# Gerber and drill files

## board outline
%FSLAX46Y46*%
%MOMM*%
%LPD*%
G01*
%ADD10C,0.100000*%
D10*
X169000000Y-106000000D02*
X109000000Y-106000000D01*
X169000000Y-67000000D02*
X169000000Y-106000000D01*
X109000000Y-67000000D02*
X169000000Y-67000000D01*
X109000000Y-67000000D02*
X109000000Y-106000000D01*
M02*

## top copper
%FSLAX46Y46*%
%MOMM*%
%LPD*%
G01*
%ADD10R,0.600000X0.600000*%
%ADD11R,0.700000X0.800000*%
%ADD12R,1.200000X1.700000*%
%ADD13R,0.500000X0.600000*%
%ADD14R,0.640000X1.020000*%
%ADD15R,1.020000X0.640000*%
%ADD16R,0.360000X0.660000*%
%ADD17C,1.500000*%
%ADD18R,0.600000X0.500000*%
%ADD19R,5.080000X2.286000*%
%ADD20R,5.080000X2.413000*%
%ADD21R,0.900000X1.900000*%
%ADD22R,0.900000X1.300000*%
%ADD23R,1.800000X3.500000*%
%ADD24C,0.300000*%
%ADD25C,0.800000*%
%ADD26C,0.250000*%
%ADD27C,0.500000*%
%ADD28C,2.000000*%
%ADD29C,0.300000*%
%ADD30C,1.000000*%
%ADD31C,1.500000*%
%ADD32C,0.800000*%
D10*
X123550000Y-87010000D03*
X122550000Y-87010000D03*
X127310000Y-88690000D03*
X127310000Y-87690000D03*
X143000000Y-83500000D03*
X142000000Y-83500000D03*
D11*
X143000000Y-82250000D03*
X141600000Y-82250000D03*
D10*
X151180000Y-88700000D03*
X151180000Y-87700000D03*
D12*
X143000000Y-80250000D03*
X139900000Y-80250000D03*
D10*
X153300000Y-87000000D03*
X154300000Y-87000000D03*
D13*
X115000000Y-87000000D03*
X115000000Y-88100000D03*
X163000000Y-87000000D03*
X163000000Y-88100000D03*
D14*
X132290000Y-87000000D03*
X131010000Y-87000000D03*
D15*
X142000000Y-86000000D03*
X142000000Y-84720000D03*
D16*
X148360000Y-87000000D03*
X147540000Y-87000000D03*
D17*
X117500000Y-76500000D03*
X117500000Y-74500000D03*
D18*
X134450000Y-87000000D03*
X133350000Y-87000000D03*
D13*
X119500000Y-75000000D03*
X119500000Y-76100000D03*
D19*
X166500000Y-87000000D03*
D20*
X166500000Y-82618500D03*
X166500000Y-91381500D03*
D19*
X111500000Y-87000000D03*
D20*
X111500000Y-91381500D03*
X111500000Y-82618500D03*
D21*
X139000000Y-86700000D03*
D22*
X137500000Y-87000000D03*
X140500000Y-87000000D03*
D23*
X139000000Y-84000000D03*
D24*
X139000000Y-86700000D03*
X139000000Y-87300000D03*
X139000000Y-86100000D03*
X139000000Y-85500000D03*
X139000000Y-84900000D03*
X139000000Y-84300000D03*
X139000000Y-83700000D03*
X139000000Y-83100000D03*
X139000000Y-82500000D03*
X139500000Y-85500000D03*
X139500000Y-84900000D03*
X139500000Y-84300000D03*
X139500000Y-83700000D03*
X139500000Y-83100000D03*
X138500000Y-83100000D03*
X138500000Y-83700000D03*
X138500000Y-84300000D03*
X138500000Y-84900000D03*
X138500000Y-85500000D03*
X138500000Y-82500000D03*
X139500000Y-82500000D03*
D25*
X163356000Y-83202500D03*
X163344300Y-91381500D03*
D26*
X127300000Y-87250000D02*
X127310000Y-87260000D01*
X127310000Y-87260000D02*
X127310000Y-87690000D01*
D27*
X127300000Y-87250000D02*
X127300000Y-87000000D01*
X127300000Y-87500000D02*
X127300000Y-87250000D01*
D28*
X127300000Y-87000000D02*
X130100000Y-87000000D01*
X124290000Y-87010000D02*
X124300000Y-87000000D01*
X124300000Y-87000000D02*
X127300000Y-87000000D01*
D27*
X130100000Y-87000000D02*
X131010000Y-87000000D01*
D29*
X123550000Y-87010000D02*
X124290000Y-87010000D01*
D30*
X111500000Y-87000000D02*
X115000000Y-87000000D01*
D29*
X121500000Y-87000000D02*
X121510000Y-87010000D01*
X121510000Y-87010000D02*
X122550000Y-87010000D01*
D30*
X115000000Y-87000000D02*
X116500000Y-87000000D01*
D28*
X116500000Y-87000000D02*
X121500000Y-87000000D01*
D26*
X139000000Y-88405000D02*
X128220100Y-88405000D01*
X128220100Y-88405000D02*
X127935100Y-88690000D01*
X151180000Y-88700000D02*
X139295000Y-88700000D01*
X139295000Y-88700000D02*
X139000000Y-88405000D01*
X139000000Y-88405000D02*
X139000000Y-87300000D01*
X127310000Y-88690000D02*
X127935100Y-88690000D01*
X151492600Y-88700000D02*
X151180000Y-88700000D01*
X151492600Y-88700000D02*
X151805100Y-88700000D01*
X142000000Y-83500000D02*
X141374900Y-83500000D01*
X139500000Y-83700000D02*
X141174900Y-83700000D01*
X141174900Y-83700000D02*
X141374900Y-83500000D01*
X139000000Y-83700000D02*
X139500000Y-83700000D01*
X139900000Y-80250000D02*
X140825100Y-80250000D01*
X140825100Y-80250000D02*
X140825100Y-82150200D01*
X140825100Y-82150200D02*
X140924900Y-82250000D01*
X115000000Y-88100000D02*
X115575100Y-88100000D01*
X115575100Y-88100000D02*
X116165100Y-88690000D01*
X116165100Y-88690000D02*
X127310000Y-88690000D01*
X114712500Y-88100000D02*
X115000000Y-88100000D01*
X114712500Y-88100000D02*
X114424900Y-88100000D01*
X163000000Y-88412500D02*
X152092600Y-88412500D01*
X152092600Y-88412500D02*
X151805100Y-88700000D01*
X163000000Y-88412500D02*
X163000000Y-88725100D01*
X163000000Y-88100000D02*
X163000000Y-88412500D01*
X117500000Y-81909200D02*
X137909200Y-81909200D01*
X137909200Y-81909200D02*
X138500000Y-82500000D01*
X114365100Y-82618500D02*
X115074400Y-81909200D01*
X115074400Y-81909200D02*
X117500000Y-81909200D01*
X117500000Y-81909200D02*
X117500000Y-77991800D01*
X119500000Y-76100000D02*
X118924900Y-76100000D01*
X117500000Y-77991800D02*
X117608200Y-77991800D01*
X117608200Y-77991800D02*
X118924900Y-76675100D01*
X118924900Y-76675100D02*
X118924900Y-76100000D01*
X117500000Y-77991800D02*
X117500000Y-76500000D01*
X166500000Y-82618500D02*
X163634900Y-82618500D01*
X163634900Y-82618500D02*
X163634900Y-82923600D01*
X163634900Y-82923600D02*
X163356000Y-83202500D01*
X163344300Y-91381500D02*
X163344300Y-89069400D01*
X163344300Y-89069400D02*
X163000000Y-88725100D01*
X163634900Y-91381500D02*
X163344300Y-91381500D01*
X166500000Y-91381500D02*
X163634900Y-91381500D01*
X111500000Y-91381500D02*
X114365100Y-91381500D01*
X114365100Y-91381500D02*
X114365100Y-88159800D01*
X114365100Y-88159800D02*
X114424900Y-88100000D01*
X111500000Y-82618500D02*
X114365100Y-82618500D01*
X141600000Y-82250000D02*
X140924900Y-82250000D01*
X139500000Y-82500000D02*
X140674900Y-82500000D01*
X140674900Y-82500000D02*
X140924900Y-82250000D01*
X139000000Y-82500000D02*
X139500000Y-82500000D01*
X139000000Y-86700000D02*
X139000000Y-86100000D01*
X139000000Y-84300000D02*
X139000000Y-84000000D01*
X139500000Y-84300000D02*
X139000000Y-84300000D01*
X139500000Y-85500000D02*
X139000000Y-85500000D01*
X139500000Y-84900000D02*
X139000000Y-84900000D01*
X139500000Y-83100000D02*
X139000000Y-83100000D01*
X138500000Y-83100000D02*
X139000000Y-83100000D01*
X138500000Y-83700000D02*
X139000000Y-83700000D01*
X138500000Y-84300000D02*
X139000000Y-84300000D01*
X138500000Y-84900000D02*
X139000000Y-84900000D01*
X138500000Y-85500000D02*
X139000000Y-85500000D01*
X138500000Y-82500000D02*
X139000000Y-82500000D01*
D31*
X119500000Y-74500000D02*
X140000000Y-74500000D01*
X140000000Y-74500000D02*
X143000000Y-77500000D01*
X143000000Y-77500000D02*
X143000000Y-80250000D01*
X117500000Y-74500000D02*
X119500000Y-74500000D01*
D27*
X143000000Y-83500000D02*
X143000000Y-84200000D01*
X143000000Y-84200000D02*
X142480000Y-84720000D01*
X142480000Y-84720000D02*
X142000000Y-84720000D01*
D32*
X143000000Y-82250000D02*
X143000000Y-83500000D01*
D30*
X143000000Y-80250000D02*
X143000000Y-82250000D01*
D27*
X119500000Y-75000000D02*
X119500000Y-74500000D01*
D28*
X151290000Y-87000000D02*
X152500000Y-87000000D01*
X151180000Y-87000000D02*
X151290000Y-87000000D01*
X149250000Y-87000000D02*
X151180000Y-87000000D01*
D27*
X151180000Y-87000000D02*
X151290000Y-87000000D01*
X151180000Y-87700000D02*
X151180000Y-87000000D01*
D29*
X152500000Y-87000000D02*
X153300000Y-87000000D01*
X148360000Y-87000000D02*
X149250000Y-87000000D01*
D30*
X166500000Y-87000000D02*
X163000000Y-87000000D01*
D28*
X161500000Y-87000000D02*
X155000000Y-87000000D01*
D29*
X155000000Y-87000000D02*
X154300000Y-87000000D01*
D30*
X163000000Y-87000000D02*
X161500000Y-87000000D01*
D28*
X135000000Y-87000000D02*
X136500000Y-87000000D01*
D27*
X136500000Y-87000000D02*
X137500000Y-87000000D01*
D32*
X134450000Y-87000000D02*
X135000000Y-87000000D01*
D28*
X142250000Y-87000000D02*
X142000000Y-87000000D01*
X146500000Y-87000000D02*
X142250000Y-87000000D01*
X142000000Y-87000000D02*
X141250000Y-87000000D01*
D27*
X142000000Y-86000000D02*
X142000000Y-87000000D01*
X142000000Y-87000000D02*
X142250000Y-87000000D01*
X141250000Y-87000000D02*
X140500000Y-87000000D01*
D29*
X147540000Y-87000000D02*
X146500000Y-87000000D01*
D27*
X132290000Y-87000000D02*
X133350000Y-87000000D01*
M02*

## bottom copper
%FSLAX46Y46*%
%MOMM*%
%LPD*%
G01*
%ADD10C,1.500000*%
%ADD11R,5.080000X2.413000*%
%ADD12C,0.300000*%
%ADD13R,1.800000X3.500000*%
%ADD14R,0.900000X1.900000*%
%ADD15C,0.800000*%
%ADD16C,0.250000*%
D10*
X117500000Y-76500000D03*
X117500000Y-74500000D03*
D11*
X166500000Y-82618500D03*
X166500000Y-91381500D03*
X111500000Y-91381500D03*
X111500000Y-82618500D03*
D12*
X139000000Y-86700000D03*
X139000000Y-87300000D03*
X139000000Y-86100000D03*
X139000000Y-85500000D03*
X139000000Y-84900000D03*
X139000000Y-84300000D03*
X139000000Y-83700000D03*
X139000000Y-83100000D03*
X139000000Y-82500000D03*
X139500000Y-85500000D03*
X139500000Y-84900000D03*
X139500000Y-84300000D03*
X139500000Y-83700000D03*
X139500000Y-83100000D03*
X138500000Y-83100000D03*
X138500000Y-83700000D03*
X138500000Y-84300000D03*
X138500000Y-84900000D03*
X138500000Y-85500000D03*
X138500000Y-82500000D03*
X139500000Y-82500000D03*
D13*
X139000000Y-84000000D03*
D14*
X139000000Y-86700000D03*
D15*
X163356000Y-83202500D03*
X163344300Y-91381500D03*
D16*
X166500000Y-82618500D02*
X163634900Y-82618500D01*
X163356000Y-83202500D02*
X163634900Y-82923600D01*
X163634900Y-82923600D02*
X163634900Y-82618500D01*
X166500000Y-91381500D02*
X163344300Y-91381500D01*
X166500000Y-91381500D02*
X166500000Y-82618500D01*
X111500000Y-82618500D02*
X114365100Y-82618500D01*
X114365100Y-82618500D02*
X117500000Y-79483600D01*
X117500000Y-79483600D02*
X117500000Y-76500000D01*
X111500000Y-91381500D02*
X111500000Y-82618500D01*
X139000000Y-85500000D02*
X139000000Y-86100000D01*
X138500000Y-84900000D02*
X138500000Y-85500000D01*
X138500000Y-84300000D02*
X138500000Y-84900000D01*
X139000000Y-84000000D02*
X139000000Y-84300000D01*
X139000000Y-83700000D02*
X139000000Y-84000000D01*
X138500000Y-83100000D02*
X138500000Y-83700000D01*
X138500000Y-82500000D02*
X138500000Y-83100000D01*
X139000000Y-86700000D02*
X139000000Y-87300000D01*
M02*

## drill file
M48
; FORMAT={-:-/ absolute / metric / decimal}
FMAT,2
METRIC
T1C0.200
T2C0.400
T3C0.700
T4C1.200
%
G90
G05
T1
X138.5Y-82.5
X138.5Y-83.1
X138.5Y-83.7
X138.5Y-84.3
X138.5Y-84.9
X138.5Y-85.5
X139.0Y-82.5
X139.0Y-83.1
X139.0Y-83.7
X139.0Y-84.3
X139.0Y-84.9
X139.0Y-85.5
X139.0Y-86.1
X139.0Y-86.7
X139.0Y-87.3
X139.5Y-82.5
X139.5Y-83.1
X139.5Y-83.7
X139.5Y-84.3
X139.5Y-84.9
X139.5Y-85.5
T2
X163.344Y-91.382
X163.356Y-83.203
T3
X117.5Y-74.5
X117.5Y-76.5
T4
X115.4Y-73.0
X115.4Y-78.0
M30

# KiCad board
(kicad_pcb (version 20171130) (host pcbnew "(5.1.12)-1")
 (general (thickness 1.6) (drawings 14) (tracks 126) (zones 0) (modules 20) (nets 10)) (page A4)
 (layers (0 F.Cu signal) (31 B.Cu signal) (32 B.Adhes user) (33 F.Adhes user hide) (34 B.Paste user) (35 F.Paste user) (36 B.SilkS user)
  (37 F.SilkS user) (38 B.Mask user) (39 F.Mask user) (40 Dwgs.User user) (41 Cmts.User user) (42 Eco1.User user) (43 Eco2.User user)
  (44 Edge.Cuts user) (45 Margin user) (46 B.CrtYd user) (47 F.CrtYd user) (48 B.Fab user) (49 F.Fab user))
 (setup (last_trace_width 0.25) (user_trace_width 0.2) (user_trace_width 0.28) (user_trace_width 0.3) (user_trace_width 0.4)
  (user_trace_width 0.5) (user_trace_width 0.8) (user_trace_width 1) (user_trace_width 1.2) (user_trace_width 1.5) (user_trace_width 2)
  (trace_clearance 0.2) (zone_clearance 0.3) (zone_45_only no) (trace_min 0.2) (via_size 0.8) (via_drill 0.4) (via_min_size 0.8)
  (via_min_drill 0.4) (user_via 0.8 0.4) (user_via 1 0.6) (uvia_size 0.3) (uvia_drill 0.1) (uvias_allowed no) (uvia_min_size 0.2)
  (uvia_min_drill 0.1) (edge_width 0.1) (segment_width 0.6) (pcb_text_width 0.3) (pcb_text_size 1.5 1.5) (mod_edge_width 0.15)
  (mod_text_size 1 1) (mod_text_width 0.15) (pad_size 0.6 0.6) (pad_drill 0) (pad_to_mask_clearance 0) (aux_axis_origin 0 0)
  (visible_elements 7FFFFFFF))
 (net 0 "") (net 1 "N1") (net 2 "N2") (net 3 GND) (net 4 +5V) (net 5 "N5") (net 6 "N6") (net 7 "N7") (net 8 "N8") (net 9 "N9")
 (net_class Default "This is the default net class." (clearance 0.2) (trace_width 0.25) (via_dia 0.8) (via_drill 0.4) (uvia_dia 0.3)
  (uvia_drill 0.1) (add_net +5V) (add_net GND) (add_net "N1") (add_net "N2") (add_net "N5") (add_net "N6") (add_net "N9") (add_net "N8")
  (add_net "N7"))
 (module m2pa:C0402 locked (layer F.Cu) (at 123.55 87.01 180)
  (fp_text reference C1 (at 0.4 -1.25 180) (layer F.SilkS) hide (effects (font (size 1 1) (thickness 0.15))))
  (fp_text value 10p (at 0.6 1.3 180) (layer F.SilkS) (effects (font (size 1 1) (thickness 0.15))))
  (pad 1 smd rect (at 0 0 180) (size 0.6 0.6) (layers F.Cu F.Paste F.Mask) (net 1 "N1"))
  (pad 2 smd rect (at 1 0 180) (size 0.6 0.6) (layers F.Cu F.Paste F.Mask) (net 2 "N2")))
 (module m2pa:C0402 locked (layer F.Cu) (at 127.31 88.69 90)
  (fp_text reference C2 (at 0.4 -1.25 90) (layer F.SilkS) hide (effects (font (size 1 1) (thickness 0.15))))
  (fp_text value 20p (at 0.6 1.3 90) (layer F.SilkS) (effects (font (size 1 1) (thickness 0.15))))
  (pad 1 smd rect (at 0 0 90) (size 0.6 0.6) (layers F.Cu F.Paste F.Mask) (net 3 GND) (zone_connect 2))
  (pad 2 smd rect (at 1 0 90) (size 0.6 0.6) (layers F.Cu F.Paste F.Mask) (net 1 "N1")))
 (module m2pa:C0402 (layer F.Cu) (at 143 83.5 180)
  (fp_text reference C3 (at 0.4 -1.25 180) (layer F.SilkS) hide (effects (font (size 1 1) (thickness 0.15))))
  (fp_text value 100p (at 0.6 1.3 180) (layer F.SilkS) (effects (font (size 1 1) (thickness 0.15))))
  (pad 1 smd rect (at 0 0 180) (size 0.6 0.6) (layers F.Cu F.Paste F.Mask) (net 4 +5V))
  (pad 2 smd rect (at 1 0 180) (size 0.6 0.6) (layers F.Cu F.Paste F.Mask) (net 3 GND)))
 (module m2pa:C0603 (layer F.Cu) (at 143 82.25 180)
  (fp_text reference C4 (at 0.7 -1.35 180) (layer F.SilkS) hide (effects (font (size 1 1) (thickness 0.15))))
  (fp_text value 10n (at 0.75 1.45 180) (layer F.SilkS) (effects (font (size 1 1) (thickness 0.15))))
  (pad 1 smd rect (at 0 0 180) (size 0.7 0.8) (layers F.Cu F.Paste F.Mask) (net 4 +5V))
  (pad 2 smd rect (at 1.4 0 180) (size 0.7 0.8) (layers F.Cu F.Paste F.Mask) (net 3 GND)))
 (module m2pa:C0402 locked (layer F.Cu) (at 151.18 88.7 90)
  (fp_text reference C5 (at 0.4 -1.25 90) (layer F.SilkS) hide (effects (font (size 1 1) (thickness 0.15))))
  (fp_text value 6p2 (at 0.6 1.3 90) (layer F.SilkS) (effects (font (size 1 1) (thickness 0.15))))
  (pad 1 smd rect (at 0 0 90) (size 0.6 0.6) (layers F.Cu F.Paste F.Mask) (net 3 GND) (zone_connect 2))
  (pad 2 smd rect (at 1 0 90) (size 0.6 0.6) (layers F.Cu F.Paste F.Mask) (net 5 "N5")))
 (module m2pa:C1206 (layer F.Cu) (at 143 80.25 180)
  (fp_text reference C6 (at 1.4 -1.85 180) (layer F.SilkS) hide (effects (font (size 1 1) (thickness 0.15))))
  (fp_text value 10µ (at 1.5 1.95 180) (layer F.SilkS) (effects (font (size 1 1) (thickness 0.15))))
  (pad 1 smd rect (at 0 0 180) (size 1.2 1.7) (layers F.Cu F.Paste F.Mask) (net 4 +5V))
  (pad 2 smd rect (at 3.1 0 180) (size 1.2 1.7) (layers F.Cu F.Paste F.Mask) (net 3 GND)))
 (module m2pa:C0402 (layer F.Cu) (at 153.3 87)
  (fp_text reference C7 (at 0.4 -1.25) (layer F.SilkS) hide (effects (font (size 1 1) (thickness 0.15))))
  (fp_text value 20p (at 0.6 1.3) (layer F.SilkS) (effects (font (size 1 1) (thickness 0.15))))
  (pad 1 smd rect (at 0 0) (size 0.6 0.6) (layers F.Cu F.Paste F.Mask) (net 5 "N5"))
  (pad 2 smd rect (at 1 0) (size 0.6 0.6) (layers F.Cu F.Paste F.Mask) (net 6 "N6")))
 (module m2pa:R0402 (layer F.Cu) (at 115 87 270)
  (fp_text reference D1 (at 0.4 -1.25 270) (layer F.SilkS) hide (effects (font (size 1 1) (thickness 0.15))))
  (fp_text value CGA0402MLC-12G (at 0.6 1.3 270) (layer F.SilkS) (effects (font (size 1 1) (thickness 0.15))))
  (pad 1 smd rect (at 0 0 270) (size 0.6 0.5) (layers F.Cu F.Paste F.Mask) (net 2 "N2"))
  (pad 2 smd rect (at 1.1 0 270) (size 0.6 0.5) (layers F.Cu F.Paste F.Mask) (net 3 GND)))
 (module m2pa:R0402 (layer F.Cu) (at 163 87 270)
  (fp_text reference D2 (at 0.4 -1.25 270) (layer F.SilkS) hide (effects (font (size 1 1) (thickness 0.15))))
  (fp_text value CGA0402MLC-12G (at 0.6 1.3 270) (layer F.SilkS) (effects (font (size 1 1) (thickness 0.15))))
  (pad 1 smd rect (at 0 0 270) (size 0.6 0.5) (layers F.Cu F.Paste F.Mask) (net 6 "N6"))
  (pad 2 smd rect (at 1.1 0 270) (size 0.6 0.5) (layers F.Cu F.Paste F.Mask) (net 3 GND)))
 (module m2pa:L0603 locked (layer F.Cu) (at 132.29 87 180)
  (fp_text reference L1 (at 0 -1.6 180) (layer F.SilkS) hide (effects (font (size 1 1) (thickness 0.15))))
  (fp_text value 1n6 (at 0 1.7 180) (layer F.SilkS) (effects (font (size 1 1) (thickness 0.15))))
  (pad 1 smd rect (at 0 0 180) (size 0.64 1.02) (layers F.Cu F.Paste F.Mask) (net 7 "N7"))
  (pad 2 smd rect (at 1.28 0 180) (size 0.64 1.02) (layers F.Cu F.Paste F.Mask) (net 1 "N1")))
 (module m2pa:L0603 (layer F.Cu) (at 142 86 90)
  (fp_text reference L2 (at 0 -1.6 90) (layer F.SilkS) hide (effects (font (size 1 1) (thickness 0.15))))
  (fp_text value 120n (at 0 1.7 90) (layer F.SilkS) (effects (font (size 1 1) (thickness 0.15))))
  (pad 1 smd rect (at 0 0 90) (size 0.64 1.02) (layers F.Cu F.Paste F.Mask) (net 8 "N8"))
  (pad 2 smd rect (at 1.28 0 90) (size 0.64 1.02) (layers F.Cu F.Paste F.Mask) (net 4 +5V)))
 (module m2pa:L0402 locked (layer F.Cu) (at 148.36 87 180)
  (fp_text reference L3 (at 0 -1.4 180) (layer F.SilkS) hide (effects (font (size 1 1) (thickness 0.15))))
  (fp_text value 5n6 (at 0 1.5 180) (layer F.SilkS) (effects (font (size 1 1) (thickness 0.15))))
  (pad 1 smd rect (at 0 0 180) (size 0.36 0.66) (layers F.Cu F.Paste F.Mask) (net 5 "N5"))
  (pad 2 smd rect (at 0.82 0 180) (size 0.36 0.66) (layers F.Cu F.Paste F.Mask) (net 8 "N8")))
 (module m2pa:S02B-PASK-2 (layer F.Cu) (at 117.5 76.5 90)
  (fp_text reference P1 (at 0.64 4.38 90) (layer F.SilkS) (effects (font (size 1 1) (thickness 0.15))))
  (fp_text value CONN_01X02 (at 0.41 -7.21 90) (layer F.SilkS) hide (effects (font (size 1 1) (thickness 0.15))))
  (pad 1 thru_hole circle (at 0 0 90) (size 1.5 1.5) (drill 0.7) (layers *.Cu *.Mask F.SilkS) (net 3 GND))
  (pad 2 thru_hole circle (at 2 0 90) (size 1.5 1.5) (drill 0.7) (layers *.Cu *.Mask F.SilkS) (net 4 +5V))
  (pad "" np_thru_hole circle (at -1.5 -2.1 90) (size 1.2 1.2) (drill 1.2) (layers *.Cu *.Mask F.SilkS))
  (pad "" np_thru_hole circle (at 3.5 -2.1 90) (size 1.2 1.2) (drill 1.2) (layers *.Cu *.Mask F.SilkS)))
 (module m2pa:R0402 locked (layer F.Cu) (at 134.45 87 180)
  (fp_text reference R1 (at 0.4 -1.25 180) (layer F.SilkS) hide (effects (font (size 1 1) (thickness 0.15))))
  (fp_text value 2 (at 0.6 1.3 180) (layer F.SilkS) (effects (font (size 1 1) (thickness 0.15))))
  (pad 1 smd rect (at 0 0 180) (size 0.6 0.5) (layers F.Cu F.Paste F.Mask) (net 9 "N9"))
  (pad 2 smd rect (at 1.1 0 180) (size 0.6 0.5) (layers F.Cu F.Paste F.Mask) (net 7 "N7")))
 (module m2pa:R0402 (layer F.Cu) (at 119.5 75 270)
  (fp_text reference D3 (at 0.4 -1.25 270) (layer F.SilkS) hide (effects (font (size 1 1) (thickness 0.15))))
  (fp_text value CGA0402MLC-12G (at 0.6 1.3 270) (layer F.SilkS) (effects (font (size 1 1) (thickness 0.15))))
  (pad 1 smd rect (at 0 0 270) (size 0.6 0.5) (layers F.Cu F.Paste F.Mask) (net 4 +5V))
  (pad 2 smd rect (at 1.1 0 270) (size 0.6 0.5) (layers F.Cu F.Paste F.Mask) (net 3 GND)))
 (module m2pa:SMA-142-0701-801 (layer F.Cu) (at 166.5 87 270)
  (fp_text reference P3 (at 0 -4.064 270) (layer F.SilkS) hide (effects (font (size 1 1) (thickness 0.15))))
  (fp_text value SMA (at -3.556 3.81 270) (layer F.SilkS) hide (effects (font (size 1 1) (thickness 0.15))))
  (pad 1 smd rect (at 0 0 270) (size 2.286 5.08) (layers F.Cu F.Mask) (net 6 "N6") (zone_connect 2))
  (pad 2 smd rect (at -4.3815 0 270) (size 2.413 5.08) (layers F.Cu F.Mask) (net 3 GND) (zone_connect 2))
  (pad 3 smd rect (at 4.3815 0 270) (size 2.413 5.08) (layers F.Cu F.Mask) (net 3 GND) (zone_connect 2))
  (pad 4 smd rect (at -4.3815 0 270) (size 2.413 5.08) (layers B.Cu B.Mask) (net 3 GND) (zone_connect 2))
  (pad 5 smd rect (at 4.3815 0 270) (size 2.413 5.08) (layers B.Cu B.Mask) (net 3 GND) (zone_connect 2)))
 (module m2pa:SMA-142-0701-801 (layer F.Cu) (at 111.5 87 90)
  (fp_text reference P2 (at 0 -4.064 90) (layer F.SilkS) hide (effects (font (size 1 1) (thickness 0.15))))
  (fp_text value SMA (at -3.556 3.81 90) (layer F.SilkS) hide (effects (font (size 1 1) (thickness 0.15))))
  (pad 1 smd rect (at 0 0 90) (size 2.286 5.08) (layers F.Cu F.Mask) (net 2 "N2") (zone_connect 2))
  (pad 2 smd rect (at -4.3815 0 90) (size 2.413 5.08) (layers F.Cu F.Mask) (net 3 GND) (zone_connect 2))
  (pad 3 smd rect (at 4.3815 0 90) (size 2.413 5.08) (layers F.Cu F.Mask) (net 3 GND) (zone_connect 2))
  (pad 4 smd rect (at -4.3815 0 90) (size 2.413 5.08) (layers B.Cu B.Mask) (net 3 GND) (zone_connect 2))
  (pad 5 smd rect (at 4.3815 0 90) (size 2.413 5.08) (layers B.Cu B.Mask) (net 3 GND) (zone_connect 2)))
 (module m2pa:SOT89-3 (layer F.Cu) (at 139 87)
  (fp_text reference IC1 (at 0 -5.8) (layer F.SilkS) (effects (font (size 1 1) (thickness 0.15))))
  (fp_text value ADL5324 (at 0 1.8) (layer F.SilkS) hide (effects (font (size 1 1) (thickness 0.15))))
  (pad 2 smd rect (at 0 -0.3 180) (size 0.9 1.9) (layers F.Cu F.Paste F.Mask) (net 3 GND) (zone_connect 2))
  (pad 1 smd rect (at -1.5 0 180) (size 0.9 1.3) (layers F.Cu F.Paste F.Mask) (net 9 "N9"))
  (pad 3 smd rect (at 1.5 0 180) (size 0.9 1.3) (layers F.Cu F.Paste F.Mask) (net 8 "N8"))
  (pad 2 smd rect (at 0 -3 180) (size 1.8 3.5) (layers F.Cu F.Paste F.Mask) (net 3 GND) (zone_connect 2))
  (pad 2 thru_hole circle (at 0 -0.3 180) (size 0.3 0.3) (drill 0.2) (layers *.Cu F.SilkS F.Mask) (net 3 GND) (zone_connect 2))
  (pad 2 thru_hole circle (at 0 0.3 180) (size 0.3 0.3) (drill 0.2) (layers *.Cu F.SilkS F.Mask) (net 3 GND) (zone_connect 2))
  (pad 2 thru_hole circle (at 0 -0.9 180) (size 0.3 0.3) (drill 0.2) (layers *.Cu F.SilkS F.Mask) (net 3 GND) (zone_connect 2))
  (pad 2 thru_hole circle (at 0 -1.5 180) (size 0.3 0.3) (drill 0.2) (layers *.Cu F.SilkS F.Mask) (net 3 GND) (zone_connect 2))
  (pad 2 thru_hole circle (at 0 -2.1 180) (size 0.3 0.3) (drill 0.2) (layers *.Cu F.SilkS F.Mask) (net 3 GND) (zone_connect 2))
  (pad 2 thru_hole circle (at 0 -2.7 180) (size 0.3 0.3) (drill 0.2) (layers *.Cu F.SilkS F.Mask) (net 3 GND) (zone_connect 2))
  (pad 2 thru_hole circle (at 0 -3.3 180) (size 0.3 0.3) (drill 0.2) (layers *.Cu F.SilkS F.Mask) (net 3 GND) (zone_connect 2))
  (pad 2 thru_hole circle (at 0 -3.9 180) (size 0.3 0.3) (drill 0.2) (layers *.Cu F.SilkS F.Mask) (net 3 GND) (zone_connect 2))
  (pad 2 thru_hole circle (at 0 -4.5 180) (size 0.3 0.3) (drill 0.2) (layers *.Cu F.SilkS F.Mask) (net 3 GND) (zone_connect 2))
  (pad 2 thru_hole circle (at 0.5 -1.5 180) (size 0.3 0.3) (drill 0.2) (layers *.Cu F.SilkS F.Mask) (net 3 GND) (zone_connect 2))
  (pad 2 thru_hole circle (at 0.5 -2.1 180) (size 0.3 0.3) (drill 0.2) (layers *.Cu F.SilkS F.Mask) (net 3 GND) (zone_connect 2))
  (pad 2 thru_hole circle (at 0.5 -2.7 180) (size 0.3 0.3) (drill 0.2) (layers *.Cu F.SilkS F.Mask) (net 3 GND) (zone_connect 2))
  (pad 2 thru_hole circle (at 0.5 -3.3 180) (size 0.3 0.3) (drill 0.2) (layers *.Cu F.SilkS F.Mask) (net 3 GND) (zone_connect 2))
  (pad 2 thru_hole circle (at 0.5 -3.9 180) (size 0.3 0.3) (drill 0.2) (layers *.Cu F.SilkS F.Mask) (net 3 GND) (zone_connect 2))
  (pad 2 thru_hole circle (at -0.5 -3.9 180) (size 0.3 0.3) (drill 0.2) (layers *.Cu F.SilkS F.Mask) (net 3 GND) (zone_connect 2))
  (pad 2 thru_hole circle (at -0.5 -3.3 180) (size 0.3 0.3) (drill 0.2) (layers *.Cu F.SilkS F.Mask) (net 3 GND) (zone_connect 2))
  (pad 2 thru_hole circle (at -0.5 -2.7 180) (size 0.3 0.3) (drill 0.2) (layers *.Cu F.SilkS F.Mask) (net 3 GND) (zone_connect 2))
  (pad 2 thru_hole circle (at -0.5 -2.1 180) (size 0.3 0.3) (drill 0.2) (layers *.Cu F.SilkS F.Mask) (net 3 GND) (zone_connect 2))
  (pad 2 thru_hole circle (at -0.5 -1.5 180) (size 0.3 0.3) (drill 0.2) (layers *.Cu F.SilkS F.Mask) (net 3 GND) (zone_connect 2))
  (pad 2 thru_hole circle (at -0.5 -4.5 180) (size 0.3 0.3) (drill 0.2) (layers *.Cu F.SilkS F.Mask) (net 3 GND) (zone_connect 2))
  (pad 2 thru_hole circle (at 0.5 -4.5 180) (size 0.3 0.3) (drill 0.2) (layers *.Cu F.SilkS F.Mask) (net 3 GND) (zone_connect 2))
  (pad 2 smd rect (at 0 -3 180) (size 1.8 3.5) (layers B.Cu) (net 3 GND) (zone_connect 2))
  (pad 2 smd rect (at 0 -0.3 180) (size 0.9 1.9) (layers B.Cu) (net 3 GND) (zone_connect 2)))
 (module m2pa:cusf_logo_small (layer F.Cu) (at 116 98)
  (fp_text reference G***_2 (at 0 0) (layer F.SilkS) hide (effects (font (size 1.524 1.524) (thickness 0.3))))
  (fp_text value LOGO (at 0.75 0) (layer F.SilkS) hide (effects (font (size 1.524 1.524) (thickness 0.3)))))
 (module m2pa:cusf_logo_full (layer F.Cu) (at 140.5 87.5)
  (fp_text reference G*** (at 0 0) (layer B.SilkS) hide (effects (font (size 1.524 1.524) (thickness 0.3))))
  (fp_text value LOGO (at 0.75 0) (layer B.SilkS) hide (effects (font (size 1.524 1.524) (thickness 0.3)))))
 (gr_line (start 169 106) (end 109 106) (angle 90) (layer Edge.Cuts) (width 0.1))
 (gr_line (start 169 67) (end 169 106) (angle 90) (layer Edge.Cuts) (width 0.1))
 (gr_line (start 109 67) (end 169 67) (angle 90) (layer Edge.Cuts) (width 0.1))
 (gr_line (start 109 67) (end 109 106) (angle 90) (layer Edge.Cuts) (width 0.1))
 (segment (start 127.3 87.25) (end 127.31 87.26) (width 0.25) (layer F.Cu) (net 1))
 (segment (start 127.31 87.26) (end 127.31 87.69) (width 0.25) (layer F.Cu) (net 1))
 (segment (start 127.3 87.25) (end 127.3 87) (width 0.5) (layer F.Cu) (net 1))
 (segment (start 127.3 87.5) (end 127.3 87.25) (width 0.5) (layer F.Cu) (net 1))
 (segment (start 127.3 87) (end 130.1 87) (width 2) (layer F.Cu) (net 1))
 (segment (start 124.29 87.01) (end 124.3 87) (width 2) (layer F.Cu) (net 1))
 (segment (start 124.3 87) (end 127.3 87) (width 2) (layer F.Cu) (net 1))
 (segment (start 130.1 87) (end 131.01 87) (width 0.5) (layer F.Cu) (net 1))
 (segment (start 123.55 87.01) (end 124.29 87.01) (width 0.3) (layer F.Cu) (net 1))
 (segment (start 111.5 87) (end 115 87) (width 1) (layer F.Cu) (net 2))
 (segment (start 121.5 87) (end 121.51 87.01) (width 0.3) (layer F.Cu) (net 2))
 (segment (start 121.51 87.01) (end 122.55 87.01) (width 0.3) (layer F.Cu) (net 2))
 (segment (start 115 87) (end 116.5 87) (width 1) (layer F.Cu) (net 2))
 (segment (start 116.5 87) (end 121.5 87) (width 2) (layer F.Cu) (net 2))
 (segment (start 139 88.405) (end 128.2201 88.405) (width 0.25) (layer F.Cu) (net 3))
 (segment (start 128.2201 88.405) (end 127.9351 88.69) (width 0.25) (layer F.Cu) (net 3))
 (segment (start 151.18 88.7) (end 139.295 88.7) (width 0.25) (layer F.Cu) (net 3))
 (segment (start 139.295 88.7) (end 139 88.405) (width 0.25) (layer F.Cu) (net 3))
 (segment (start 139 88.405) (end 139 87.3) (width 0.25) (layer F.Cu) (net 3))
 (segment (start 127.31 88.69) (end 127.9351 88.69) (width 0.25) (layer F.Cu) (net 3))
 (segment (start 151.4926 88.7) (end 151.18 88.7) (width 0.25) (layer F.Cu) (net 3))
 (segment (start 151.4926 88.7) (end 151.8051 88.7) (width 0.25) (layer F.Cu) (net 3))
 (segment (start 142 83.5) (end 141.3749 83.5) (width 0.25) (layer F.Cu) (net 3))
 (segment (start 139.5 83.7) (end 141.1749 83.7) (width 0.25) (layer F.Cu) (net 3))
 (segment (start 141.1749 83.7) (end 141.3749 83.5) (width 0.25) (layer F.Cu) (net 3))
 (segment (start 139 83.7) (end 139.5 83.7) (width 0.25) (layer F.Cu) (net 3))
 (segment (start 139.9 80.25) (end 140.8251 80.25) (width 0.25) (layer F.Cu) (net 3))
 (segment (start 140.8251 80.25) (end 140.8251 82.1502) (width 0.25) (layer F.Cu) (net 3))
 (segment (start 140.8251 82.1502) (end 140.9249 82.25) (width 0.25) (layer F.Cu) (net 3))
 (segment (start 115 88.1) (end 115.5751 88.1) (width 0.25) (layer F.Cu) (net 3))
 (segment (start 115.5751 88.1) (end 116.1651 88.69) (width 0.25) (layer F.Cu) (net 3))
 (segment (start 116.1651 88.69) (end 127.31 88.69) (width 0.25) (layer F.Cu) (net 3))
 (segment (start 114.7125 88.1) (end 115 88.1) (width 0.25) (layer F.Cu) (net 3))
 (segment (start 114.7125 88.1) (end 114.4249 88.1) (width 0.25) (layer F.Cu) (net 3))
 (segment (start 163 88.4125) (end 152.0926 88.4125) (width 0.25) (layer F.Cu) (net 3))
 (segment (start 152.0926 88.4125) (end 151.8051 88.7) (width 0.25) (layer F.Cu) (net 3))
 (segment (start 163 88.4125) (end 163 88.7251) (width 0.25) (layer F.Cu) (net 3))
 (segment (start 163 88.1) (end 163 88.4125) (width 0.25) (layer F.Cu) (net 3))
 (segment (start 117.5 81.9092) (end 137.9092 81.9092) (width 0.25) (layer F.Cu) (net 3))
 (segment (start 137.9092 81.9092) (end 138.5 82.5) (width 0.25) (layer F.Cu) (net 3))
 (segment (start 114.3651 82.6185) (end 115.0744 81.9092) (width 0.25) (layer F.Cu) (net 3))
 (segment (start 115.0744 81.9092) (end 117.5 81.9092) (width 0.25) (layer F.Cu) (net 3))
 (segment (start 117.5 81.9092) (end 117.5 77.9918) (width 0.25) (layer F.Cu) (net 3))
 (segment (start 119.5 76.1) (end 118.9249 76.1) (width 0.25) (layer F.Cu) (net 3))
 (segment (start 117.5 77.9918) (end 117.6082 77.9918) (width 0.25) (layer F.Cu) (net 3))
 (segment (start 117.6082 77.9918) (end 118.9249 76.6751) (width 0.25) (layer F.Cu) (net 3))
 (segment (start 118.9249 76.6751) (end 118.9249 76.1) (width 0.25) (layer F.Cu) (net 3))
 (segment (start 117.5 77.9918) (end 117.5 76.5) (width 0.25) (layer F.Cu) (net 3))
 (segment (start 166.5 82.6185) (end 163.6349 82.6185) (width 0.25) (layer F.Cu) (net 3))
 (segment (start 166.5 82.6185) (end 163.6349 82.6185) (width 0.25) (layer B.Cu) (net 3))
 (segment (start 163.6349 82.6185) (end 163.6349 82.9236) (width 0.25) (layer F.Cu) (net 3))
 (segment (start 163.6349 82.9236) (end 163.356 83.2025) (width 0.25) (layer F.Cu) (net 3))
 (segment (start 163.356 83.2025) (end 163.6349 82.9236) (width 0.25) (layer B.Cu) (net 3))
 (segment (start 163.6349 82.9236) (end 163.6349 82.6185) (width 0.25) (layer B.Cu) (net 3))
 (segment (start 163.3443 91.3815) (end 163.3443 89.0694) (width 0.25) (layer F.Cu) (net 3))
 (segment (start 163.3443 89.0694) (end 163 88.7251) (width 0.25) (layer F.Cu) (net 3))
 (segment (start 163.6349 91.3815) (end 163.3443 91.3815) (width 0.25) (layer F.Cu) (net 3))
 (segment (start 166.5 91.3815) (end 163.3443 91.3815) (width 0.25) (layer B.Cu) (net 3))
 (segment (start 166.5 91.3815) (end 166.5 82.6185) (width 0.25) (layer B.Cu) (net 3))
 (segment (start 166.5 91.3815) (end 163.6349 91.3815) (width 0.25) (layer F.Cu) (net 3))
 (segment (start 111.5 91.3815) (end 114.3651 91.3815) (width 0.25) (layer F.Cu) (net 3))
 (segment (start 114.3651 91.3815) (end 114.3651 88.1598) (width 0.25) (layer F.Cu) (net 3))
 (segment (start 114.3651 88.1598) (end 114.4249 88.1) (width 0.25) (layer F.Cu) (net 3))
 (segment (start 111.5 82.6185) (end 114.3651 82.6185) (width 0.25) (layer F.Cu) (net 3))
 (segment (start 111.5 82.6185) (end 114.3651 82.6185) (width 0.25) (layer B.Cu) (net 3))
 (segment (start 114.3651 82.6185) (end 117.5 79.4836) (width 0.25) (layer B.Cu) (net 3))
 (segment (start 117.5 79.4836) (end 117.5 76.5) (width 0.25) (layer B.Cu) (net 3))
 (segment (start 111.5 91.3815) (end 111.5 82.6185) (width 0.25) (layer B.Cu) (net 3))
 (segment (start 141.6 82.25) (end 140.9249 82.25) (width 0.25) (layer F.Cu) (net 3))
 (segment (start 139.5 82.5) (end 140.6749 82.5) (width 0.25) (layer F.Cu) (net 3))
 (segment (start 140.6749 82.5) (end 140.9249 82.25) (width 0.25) (layer F.Cu) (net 3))
 (segment (start 139 82.5) (end 139.5 82.5) (width 0.25) (layer F.Cu) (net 3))
 (segment (start 139 86.7) (end 139 86.1) (width 0.25) (layer F.Cu) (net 3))
 (segment (start 139 84.3) (end 139 84) (width 0.25) (layer F.Cu) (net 3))
 (segment (start 139.5 84.3) (end 139 84.3) (width 0.25) (layer F.Cu) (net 3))
 (segment (start 139 85.5) (end 139 86.1) (width 0.25) (layer B.Cu) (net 3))
 (segment (start 138.5 84.9) (end 138.5 85.5) (width 0.25) (layer B.Cu) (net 3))
 (segment (start 138.5 84.3) (end 138.5 84.9) (width 0.25) (layer B.Cu) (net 3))
 (segment (start 139 84) (end 139 84.3) (width 0.25) (layer B.Cu) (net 3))
 (segment (start 139 83.7) (end 139 84) (width 0.25) (layer B.Cu) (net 3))
 (segment (start 138.5 83.1) (end 138.5 83.7) (width 0.25) (layer B.Cu) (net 3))
 (segment (start 138.5 82.5) (end 138.5 83.1) (width 0.25) (layer B.Cu) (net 3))
 (segment (start 139.5 85.5) (end 139 85.5) (width 0.25) (layer F.Cu) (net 3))
 (segment (start 139.5 84.9) (end 139 84.9) (width 0.25) (layer F.Cu) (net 3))
 (segment (start 139.5 83.1) (end 139 83.1) (width 0.25) (layer F.Cu) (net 3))
 (segment (start 138.5 83.1) (end 139 83.1) (width 0.25) (layer F.Cu) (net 3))
 (segment (start 138.5 83.7) (end 139 83.7) (width 0.25) (layer F.Cu) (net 3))
 (segment (start 138.5 84.3) (end 139 84.3) (width 0.25) (layer F.Cu) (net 3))
 (segment (start 138.5 84.9) (end 139 84.9) (width 0.25) (layer F.Cu) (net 3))
 (segment (start 138.5 85.5) (end 139 85.5) (width 0.25) (layer F.Cu) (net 3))
 (segment (start 138.5 82.5) (end 139 82.5) (width 0.25) (layer F.Cu) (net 3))
 (segment (start 139 86.7) (end 139 87.3) (width 0.25) (layer B.Cu) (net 3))
 (via (at 163.356 83.2025) (size 0.8) (layers F.Cu B.Cu) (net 3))
 (via (at 163.3443 91.3815) (size 0.8) (layers F.Cu B.Cu) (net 3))
 (segment (start 119.5 74.5) (end 140 74.5) (width 1.5) (layer F.Cu) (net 4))
 (segment (start 140 74.5) (end 143 77.5) (width 1.5) (layer F.Cu) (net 4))
 (segment (start 143 77.5) (end 143 80.25) (width 1.5) (layer F.Cu) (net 4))
 (segment (start 117.5 74.5) (end 119.5 74.5) (width 1.5) (layer F.Cu) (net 4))
 (segment (start 143 83.5) (end 143 84.2) (width 0.5) (layer F.Cu) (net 4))
 (segment (start 143 84.2) (end 142.48 84.72) (width 0.5) (layer F.Cu) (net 4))
 (segment (start 142.48 84.72) (end 142 84.72) (width 0.5) (layer F.Cu) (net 4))
 (segment (start 143 82.25) (end 143 83.5) (width 0.8) (layer F.Cu) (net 4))
 (segment (start 143 80.25) (end 143 82.25) (width 1) (layer F.Cu) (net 4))
 (segment (start 119.5 75) (end 119.5 74.5) (width 0.5) (layer F.Cu) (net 4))
 (segment (start 151.29 87) (end 152.5 87) (width 2) (layer F.Cu) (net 5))
 (segment (start 151.18 87) (end 151.29 87) (width 2) (layer F.Cu) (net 5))
 (segment (start 149.25 87) (end 151.18 87) (width 2) (layer F.Cu) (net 5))
 (segment (start 151.18 87) (end 151.29 87) (width 0.5) (layer F.Cu) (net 5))
 (segment (start 151.18 87.7) (end 151.18 87) (width 0.5) (layer F.Cu) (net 5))
 (segment (start 152.5 87) (end 153.3 87) (width 0.3) (layer F.Cu) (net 5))
 (segment (start 148.36 87) (end 149.25 87) (width 0.3) (layer F.Cu) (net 5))
 (segment (start 166.5 87) (end 163 87) (width 1) (layer F.Cu) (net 6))
 (segment (start 161.5 87) (end 155 87) (width 2) (layer F.Cu) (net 6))
 (segment (start 155 87) (end 154.3 87) (width 0.3) (layer F.Cu) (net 6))
 (segment (start 163 87) (end 161.5 87) (width 1) (layer F.Cu) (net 6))
 (segment (start 135 87) (end 136.5 87) (width 2) (layer F.Cu) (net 9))
 (segment (start 136.5 87) (end 137.5 87) (width 0.5) (layer F.Cu) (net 9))
 (segment (start 134.45 87) (end 135 87) (width 0.8) (layer F.Cu) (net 9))
 (segment (start 142.25 87) (end 142 87) (width 2) (layer F.Cu) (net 8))
 (segment (start 146.5 87) (end 142.25 87) (width 2) (layer F.Cu) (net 8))
 (segment (start 142 87) (end 141.25 87) (width 2) (layer F.Cu) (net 8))
 (segment (start 142 86) (end 142 87) (width 0.5) (layer F.Cu) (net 8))
 (segment (start 142 87) (end 142.25 87) (width 0.5) (layer F.Cu) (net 8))
 (segment (start 141.25 87) (end 140.5 87) (width 0.5) (layer F.Cu) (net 8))
 (segment (start 147.54 87) (end 146.5 87) (width 0.3) (layer F.Cu) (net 8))
 (segment (start 132.29 87) (end 133.35 87) (width 0.5) (layer F.Cu) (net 7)))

